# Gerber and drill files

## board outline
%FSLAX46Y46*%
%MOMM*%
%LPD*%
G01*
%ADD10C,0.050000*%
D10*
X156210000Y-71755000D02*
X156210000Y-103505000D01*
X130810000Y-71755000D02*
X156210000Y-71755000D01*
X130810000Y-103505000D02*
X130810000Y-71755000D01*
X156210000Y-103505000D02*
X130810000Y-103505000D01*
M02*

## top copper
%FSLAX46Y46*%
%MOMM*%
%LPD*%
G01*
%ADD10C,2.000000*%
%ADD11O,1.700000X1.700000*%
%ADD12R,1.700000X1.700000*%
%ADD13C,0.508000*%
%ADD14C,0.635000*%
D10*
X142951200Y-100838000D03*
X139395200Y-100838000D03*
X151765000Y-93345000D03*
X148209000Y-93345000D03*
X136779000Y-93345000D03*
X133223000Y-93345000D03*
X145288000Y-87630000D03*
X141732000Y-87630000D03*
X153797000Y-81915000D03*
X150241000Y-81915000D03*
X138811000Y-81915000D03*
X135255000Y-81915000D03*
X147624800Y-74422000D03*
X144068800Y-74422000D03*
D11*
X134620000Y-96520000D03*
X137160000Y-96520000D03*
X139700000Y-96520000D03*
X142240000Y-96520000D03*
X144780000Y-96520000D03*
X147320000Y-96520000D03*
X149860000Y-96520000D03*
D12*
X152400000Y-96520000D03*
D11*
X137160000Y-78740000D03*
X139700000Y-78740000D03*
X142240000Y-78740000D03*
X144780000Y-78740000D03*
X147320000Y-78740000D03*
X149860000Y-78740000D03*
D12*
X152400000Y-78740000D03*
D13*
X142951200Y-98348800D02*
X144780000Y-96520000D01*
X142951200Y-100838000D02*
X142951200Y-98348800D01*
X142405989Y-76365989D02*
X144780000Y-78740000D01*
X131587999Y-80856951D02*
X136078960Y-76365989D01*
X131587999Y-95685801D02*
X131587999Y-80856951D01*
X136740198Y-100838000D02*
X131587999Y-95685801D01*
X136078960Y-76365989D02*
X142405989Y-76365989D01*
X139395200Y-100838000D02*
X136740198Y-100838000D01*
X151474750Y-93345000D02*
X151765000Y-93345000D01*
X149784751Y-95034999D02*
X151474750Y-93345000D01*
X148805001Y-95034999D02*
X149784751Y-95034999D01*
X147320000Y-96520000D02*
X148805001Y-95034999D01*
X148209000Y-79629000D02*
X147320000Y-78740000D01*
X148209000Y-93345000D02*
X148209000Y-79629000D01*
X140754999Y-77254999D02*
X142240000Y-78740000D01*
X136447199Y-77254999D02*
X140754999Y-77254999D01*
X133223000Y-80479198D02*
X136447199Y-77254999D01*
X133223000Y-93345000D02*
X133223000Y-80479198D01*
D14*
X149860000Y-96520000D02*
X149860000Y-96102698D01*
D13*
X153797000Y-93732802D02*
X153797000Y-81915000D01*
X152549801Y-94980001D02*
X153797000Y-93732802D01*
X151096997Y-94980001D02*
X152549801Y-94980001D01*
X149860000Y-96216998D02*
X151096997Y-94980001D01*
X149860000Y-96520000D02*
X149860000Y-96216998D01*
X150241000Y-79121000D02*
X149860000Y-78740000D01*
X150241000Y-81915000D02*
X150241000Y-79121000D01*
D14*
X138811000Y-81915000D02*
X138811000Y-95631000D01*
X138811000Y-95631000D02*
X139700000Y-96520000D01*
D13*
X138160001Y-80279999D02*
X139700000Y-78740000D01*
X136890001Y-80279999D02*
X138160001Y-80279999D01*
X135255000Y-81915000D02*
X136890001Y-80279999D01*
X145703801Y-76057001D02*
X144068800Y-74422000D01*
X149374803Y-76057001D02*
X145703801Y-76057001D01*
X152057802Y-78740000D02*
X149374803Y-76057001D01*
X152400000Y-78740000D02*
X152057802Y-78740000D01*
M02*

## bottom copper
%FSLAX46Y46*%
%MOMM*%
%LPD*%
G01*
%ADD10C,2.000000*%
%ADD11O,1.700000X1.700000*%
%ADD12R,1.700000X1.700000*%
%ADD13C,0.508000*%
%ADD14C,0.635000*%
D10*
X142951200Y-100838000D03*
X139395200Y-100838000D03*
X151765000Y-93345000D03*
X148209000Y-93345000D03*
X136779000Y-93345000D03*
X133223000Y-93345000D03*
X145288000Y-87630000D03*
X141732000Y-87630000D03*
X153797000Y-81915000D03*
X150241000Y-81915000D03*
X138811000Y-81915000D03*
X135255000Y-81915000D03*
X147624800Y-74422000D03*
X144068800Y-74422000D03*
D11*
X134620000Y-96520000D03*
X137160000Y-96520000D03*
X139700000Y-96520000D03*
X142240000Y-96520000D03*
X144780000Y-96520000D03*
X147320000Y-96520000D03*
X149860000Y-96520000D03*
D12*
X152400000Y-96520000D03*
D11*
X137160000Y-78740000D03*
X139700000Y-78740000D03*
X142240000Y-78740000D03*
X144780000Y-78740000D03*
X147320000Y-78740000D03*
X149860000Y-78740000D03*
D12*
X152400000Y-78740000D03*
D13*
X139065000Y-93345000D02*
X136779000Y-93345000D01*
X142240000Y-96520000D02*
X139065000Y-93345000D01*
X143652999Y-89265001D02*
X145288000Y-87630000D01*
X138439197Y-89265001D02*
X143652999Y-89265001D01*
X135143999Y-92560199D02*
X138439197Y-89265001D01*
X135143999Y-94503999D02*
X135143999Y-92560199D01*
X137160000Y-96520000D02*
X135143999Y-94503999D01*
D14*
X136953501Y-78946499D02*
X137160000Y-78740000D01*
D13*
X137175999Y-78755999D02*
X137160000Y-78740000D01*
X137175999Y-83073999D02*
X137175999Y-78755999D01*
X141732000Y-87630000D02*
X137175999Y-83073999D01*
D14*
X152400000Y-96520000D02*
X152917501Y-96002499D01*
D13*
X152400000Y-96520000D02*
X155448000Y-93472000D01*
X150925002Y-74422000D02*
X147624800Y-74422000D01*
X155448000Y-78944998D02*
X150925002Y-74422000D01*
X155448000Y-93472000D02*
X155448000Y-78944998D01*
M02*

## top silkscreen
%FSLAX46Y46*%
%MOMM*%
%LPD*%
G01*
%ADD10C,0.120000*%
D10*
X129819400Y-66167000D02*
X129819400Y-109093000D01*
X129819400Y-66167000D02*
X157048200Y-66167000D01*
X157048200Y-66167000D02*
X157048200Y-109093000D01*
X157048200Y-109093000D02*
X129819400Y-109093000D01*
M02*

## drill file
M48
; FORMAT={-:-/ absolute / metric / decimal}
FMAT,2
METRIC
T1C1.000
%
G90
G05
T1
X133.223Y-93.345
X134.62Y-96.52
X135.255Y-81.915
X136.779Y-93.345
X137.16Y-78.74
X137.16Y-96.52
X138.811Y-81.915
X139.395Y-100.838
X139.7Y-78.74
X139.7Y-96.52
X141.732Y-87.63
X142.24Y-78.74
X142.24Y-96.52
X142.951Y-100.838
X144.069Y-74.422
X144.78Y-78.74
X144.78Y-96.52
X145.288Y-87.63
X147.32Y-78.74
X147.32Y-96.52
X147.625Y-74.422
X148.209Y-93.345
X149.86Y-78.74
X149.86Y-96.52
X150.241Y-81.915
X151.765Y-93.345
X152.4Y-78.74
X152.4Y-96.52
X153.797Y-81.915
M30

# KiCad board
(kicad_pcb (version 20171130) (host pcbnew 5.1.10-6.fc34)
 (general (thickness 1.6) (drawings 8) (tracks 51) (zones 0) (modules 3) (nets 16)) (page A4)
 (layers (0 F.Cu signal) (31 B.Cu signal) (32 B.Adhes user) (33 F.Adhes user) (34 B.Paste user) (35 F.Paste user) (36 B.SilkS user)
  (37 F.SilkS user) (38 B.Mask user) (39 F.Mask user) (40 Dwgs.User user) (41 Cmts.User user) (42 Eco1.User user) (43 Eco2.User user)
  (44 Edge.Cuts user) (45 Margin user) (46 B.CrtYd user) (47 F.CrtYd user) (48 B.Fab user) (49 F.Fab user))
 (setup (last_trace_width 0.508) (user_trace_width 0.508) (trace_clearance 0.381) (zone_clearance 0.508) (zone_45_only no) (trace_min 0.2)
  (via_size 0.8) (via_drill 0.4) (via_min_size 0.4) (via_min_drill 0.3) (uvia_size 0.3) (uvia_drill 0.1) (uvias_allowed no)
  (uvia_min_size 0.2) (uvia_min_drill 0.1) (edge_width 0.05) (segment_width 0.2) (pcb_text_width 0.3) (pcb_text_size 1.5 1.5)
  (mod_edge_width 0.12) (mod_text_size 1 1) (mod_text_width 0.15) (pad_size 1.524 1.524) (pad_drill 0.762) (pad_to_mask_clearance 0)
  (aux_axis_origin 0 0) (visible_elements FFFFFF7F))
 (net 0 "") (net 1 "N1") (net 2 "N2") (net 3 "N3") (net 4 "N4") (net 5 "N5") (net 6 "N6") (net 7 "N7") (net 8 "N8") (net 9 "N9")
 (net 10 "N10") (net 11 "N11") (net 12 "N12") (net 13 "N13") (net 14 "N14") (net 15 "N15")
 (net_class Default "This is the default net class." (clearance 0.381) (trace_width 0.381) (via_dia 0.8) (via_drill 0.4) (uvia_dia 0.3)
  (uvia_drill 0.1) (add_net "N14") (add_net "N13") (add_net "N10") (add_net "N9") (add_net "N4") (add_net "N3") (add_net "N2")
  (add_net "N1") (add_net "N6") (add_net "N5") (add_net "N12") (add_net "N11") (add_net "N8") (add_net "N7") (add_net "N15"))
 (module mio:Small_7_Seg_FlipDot (layer F.Cu) (at 143.51 87.63)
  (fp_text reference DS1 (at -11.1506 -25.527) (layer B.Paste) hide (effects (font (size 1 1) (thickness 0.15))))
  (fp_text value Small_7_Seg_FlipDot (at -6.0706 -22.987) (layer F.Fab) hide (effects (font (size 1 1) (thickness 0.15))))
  (fp_line (start -13.6906 -21.463) (end -13.6906 21.463) (layer F.SilkS) (width 0.12))
  (fp_line (start -13.6906 -21.463) (end 13.5382 -21.463) (layer F.SilkS) (width 0.12))
  (fp_line (start 13.5382 -21.463) (end 13.5382 21.463) (layer F.SilkS) (width 0.12))
  (fp_line (start 13.5382 21.463) (end -13.6906 21.463) (layer F.SilkS) (width 0.12))
  (pad D2 thru_hole circle (at -0.5588 13.208) (size 2 2) (drill 1) (layers *.Cu *.Mask) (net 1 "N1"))
  (pad D1 thru_hole circle (at -4.1148 13.208) (size 2 2) (drill 1) (layers *.Cu *.Mask) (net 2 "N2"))
  (pad C2 thru_hole circle (at 8.255 5.715) (size 2 2) (drill 1) (layers *.Cu *.Mask) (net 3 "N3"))
  (pad C1 thru_hole circle (at 4.699 5.715) (size 2 2) (drill 1) (layers *.Cu *.Mask) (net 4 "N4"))
  (pad E2 thru_hole circle (at -6.731 5.715) (size 2 2) (drill 1) (layers *.Cu *.Mask) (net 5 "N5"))
  (pad E1 thru_hole circle (at -10.287 5.715) (size 2 2) (drill 1) (layers *.Cu *.Mask) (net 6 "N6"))
  (pad G2 thru_hole circle (at 1.778 0) (size 2 2) (drill 1) (layers *.Cu *.Mask) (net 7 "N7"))
  (pad G1 thru_hole circle (at -1.778 0) (size 2 2) (drill 1) (layers *.Cu *.Mask) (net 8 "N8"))
  (pad B2 thru_hole circle (at 10.287 -5.715) (size 2 2) (drill 1) (layers *.Cu *.Mask) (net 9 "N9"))
  (pad B1 thru_hole circle (at 6.731 -5.715) (size 2 2) (drill 1) (layers *.Cu *.Mask) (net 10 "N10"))
  (pad F2 thru_hole circle (at -4.699 -5.715) (size 2 2) (drill 1) (layers *.Cu *.Mask) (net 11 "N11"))
  (pad F1 thru_hole circle (at -8.255 -5.715) (size 2 2) (drill 1) (layers *.Cu *.Mask) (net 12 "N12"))
  (pad A2 thru_hole circle (at 4.1148 -13.208) (size 2 2) (drill 1) (layers *.Cu *.Mask) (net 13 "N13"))
  (pad A1 thru_hole circle (at 0.5588 -13.208) (size 2 2) (drill 1) (layers *.Cu *.Mask) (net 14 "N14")))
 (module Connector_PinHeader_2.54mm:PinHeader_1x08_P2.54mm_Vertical (layer B.Cu) (at 152.4 96.52 90)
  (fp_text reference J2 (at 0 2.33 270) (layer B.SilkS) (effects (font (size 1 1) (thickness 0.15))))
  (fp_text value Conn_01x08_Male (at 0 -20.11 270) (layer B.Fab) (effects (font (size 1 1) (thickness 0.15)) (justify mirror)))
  (pad 8 thru_hole oval (at 0 -17.78 90) (size 1.7 1.7) (drill 1) (layers *.Cu *.Mask) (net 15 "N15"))
  (pad 7 thru_hole oval (at 0 -15.24 90) (size 1.7 1.7) (drill 1) (layers *.Cu *.Mask) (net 7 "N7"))
  (pad 6 thru_hole oval (at 0 -12.7 90) (size 1.7 1.7) (drill 1) (layers *.Cu *.Mask) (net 11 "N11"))
  (pad 5 thru_hole oval (at 0 -10.16 90) (size 1.7 1.7) (drill 1) (layers *.Cu *.Mask) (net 5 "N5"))
  (pad 4 thru_hole oval (at 0 -7.62 90) (size 1.7 1.7) (drill 1) (layers *.Cu *.Mask) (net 1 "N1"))
  (pad 3 thru_hole oval (at 0 -5.08 90) (size 1.7 1.7) (drill 1) (layers *.Cu *.Mask) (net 3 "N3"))
  (pad 2 thru_hole oval (at 0 -2.54 90) (size 1.7 1.7) (drill 1) (layers *.Cu *.Mask) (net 9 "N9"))
  (pad 1 thru_hole rect (at 0 0 90) (size 1.7 1.7) (drill 1) (layers *.Cu *.Mask) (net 13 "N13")))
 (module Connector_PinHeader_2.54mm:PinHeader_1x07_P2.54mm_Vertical (layer B.Cu) (at 152.4 78.74 90)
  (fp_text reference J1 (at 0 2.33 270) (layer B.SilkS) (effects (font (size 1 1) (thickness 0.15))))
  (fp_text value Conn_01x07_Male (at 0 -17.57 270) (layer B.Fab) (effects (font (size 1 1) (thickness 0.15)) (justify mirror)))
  (pad 7 thru_hole oval (at 0 -15.24 90) (size 1.7 1.7) (drill 1) (layers *.Cu *.Mask) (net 8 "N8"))
  (pad 6 thru_hole oval (at 0 -12.7 90) (size 1.7 1.7) (drill 1) (layers *.Cu *.Mask) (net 12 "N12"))
  (pad 5 thru_hole oval (at 0 -10.16 90) (size 1.7 1.7) (drill 1) (layers *.Cu *.Mask) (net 6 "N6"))
  (pad 4 thru_hole oval (at 0 -7.62 90) (size 1.7 1.7) (drill 1) (layers *.Cu *.Mask) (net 2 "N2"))
  (pad 3 thru_hole oval (at 0 -5.08 90) (size 1.7 1.7) (drill 1) (layers *.Cu *.Mask) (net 4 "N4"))
  (pad 2 thru_hole oval (at 0 -2.54 90) (size 1.7 1.7) (drill 1) (layers *.Cu *.Mask) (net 10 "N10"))
  (pad 1 thru_hole rect (at 0 0 90) (size 1.7 1.7) (drill 1) (layers *.Cu *.Mask) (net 14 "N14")))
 (gr_line (start 156.21 71.755) (end 156.21 103.505) (layer Edge.Cuts) (width 0.05))
 (gr_line (start 130.81 71.755) (end 156.21 71.755) (layer Edge.Cuts) (width 0.05))
 (gr_line (start 130.81 103.505) (end 130.81 71.755) (layer Edge.Cuts) (width 0.05))
 (gr_line (start 156.21 103.505) (end 130.81 103.505) (layer Edge.Cuts) (width 0.05))
 (segment (start 142.9512 98.3488) (end 144.78 96.52) (width 0.508) (layer F.Cu) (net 1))
 (segment (start 142.9512 100.838) (end 142.9512 98.3488) (width 0.508) (layer F.Cu) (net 1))
 (segment (start 142.405989 76.365989) (end 144.78 78.74) (width 0.508) (layer F.Cu) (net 2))
 (segment (start 131.587999 80.856951) (end 136.07896 76.365989) (width 0.508) (layer F.Cu) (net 2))
 (segment (start 131.587999 95.685801) (end 131.587999 80.856951) (width 0.508) (layer F.Cu) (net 2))
 (segment (start 136.740198 100.838) (end 131.587999 95.685801) (width 0.508) (layer F.Cu) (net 2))
 (segment (start 136.07896 76.365989) (end 142.405989 76.365989) (width 0.508) (layer F.Cu) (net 2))
 (segment (start 139.3952 100.838) (end 136.740198 100.838) (width 0.508) (layer F.Cu) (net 2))
 (segment (start 151.47475 93.345) (end 151.765 93.345) (width 0.508) (layer F.Cu) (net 3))
 (segment (start 149.784751 95.034999) (end 151.47475 93.345) (width 0.508) (layer F.Cu) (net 3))
 (segment (start 148.805001 95.034999) (end 149.784751 95.034999) (width 0.508) (layer F.Cu) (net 3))
 (segment (start 147.32 96.52) (end 148.805001 95.034999) (width 0.508) (layer F.Cu) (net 3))
 (segment (start 148.209 79.629) (end 147.32 78.74) (width 0.508) (layer F.Cu) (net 4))
 (segment (start 148.209 93.345) (end 148.209 79.629) (width 0.508) (layer F.Cu) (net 4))
 (segment (start 139.065 93.345) (end 136.779 93.345) (width 0.508) (layer B.Cu) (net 5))
 (segment (start 142.24 96.52) (end 139.065 93.345) (width 0.508) (layer B.Cu) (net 5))
 (segment (start 140.754999 77.254999) (end 142.24 78.74) (width 0.508) (layer F.Cu) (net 6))
 (segment (start 136.447199 77.254999) (end 140.754999 77.254999) (width 0.508) (layer F.Cu) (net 6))
 (segment (start 133.223 80.479198) (end 136.447199 77.254999) (width 0.508) (layer F.Cu) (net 6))
 (segment (start 133.223 93.345) (end 133.223 80.479198) (width 0.508) (layer F.Cu) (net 6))
 (segment (start 143.652999 89.265001) (end 145.288 87.63) (width 0.508) (layer B.Cu) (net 7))
 (segment (start 138.439197 89.265001) (end 143.652999 89.265001) (width 0.508) (layer B.Cu) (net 7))
 (segment (start 135.143999 92.560199) (end 138.439197 89.265001) (width 0.508) (layer B.Cu) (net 7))
 (segment (start 135.143999 94.503999) (end 135.143999 92.560199) (width 0.508) (layer B.Cu) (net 7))
 (segment (start 137.16 96.52) (end 135.143999 94.503999) (width 0.508) (layer B.Cu) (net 7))
 (segment (start 136.953501 78.946499) (end 137.16 78.74) (width 0.635) (layer B.Cu) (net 8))
 (segment (start 137.175999 78.755999) (end 137.16 78.74) (width 0.508) (layer B.Cu) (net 8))
 (segment (start 137.175999 83.073999) (end 137.175999 78.755999) (width 0.508) (layer B.Cu) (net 8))
 (segment (start 141.732 87.63) (end 137.175999 83.073999) (width 0.508) (layer B.Cu) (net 8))
 (segment (start 149.86 96.52) (end 149.86 96.102698) (width 0.635) (layer F.Cu) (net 9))
 (segment (start 153.797 93.732802) (end 153.797 81.915) (width 0.508) (layer F.Cu) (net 9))
 (segment (start 152.549801 94.980001) (end 153.797 93.732802) (width 0.508) (layer F.Cu) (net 9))
 (segment (start 151.096997 94.980001) (end 152.549801 94.980001) (width 0.508) (layer F.Cu) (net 9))
 (segment (start 149.86 96.216998) (end 151.096997 94.980001) (width 0.508) (layer F.Cu) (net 9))
 (segment (start 149.86 96.52) (end 149.86 96.216998) (width 0.508) (layer F.Cu) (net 9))
 (segment (start 150.241 79.121) (end 149.86 78.74) (width 0.508) (layer F.Cu) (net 10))
 (segment (start 150.241 81.915) (end 150.241 79.121) (width 0.508) (layer F.Cu) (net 10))
 (segment (start 138.811 81.915) (end 138.811 95.631) (width 0.635) (layer F.Cu) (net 11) (status 10))
 (segment (start 138.811 95.631) (end 139.7 96.52) (width 0.635) (layer F.Cu) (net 11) (status 20))
 (segment (start 138.160001 80.279999) (end 139.7 78.74) (width 0.508) (layer F.Cu) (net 12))
 (segment (start 136.890001 80.279999) (end 138.160001 80.279999) (width 0.508) (layer F.Cu) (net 12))
 (segment (start 135.255 81.915) (end 136.890001 80.279999) (width 0.508) (layer F.Cu) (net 12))
 (segment (start 152.4 96.52) (end 152.917501 96.002499) (width 0.635) (layer B.Cu) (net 13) (status 30))
 (segment (start 152.4 96.52) (end 155.448 93.472) (width 0.508) (layer B.Cu) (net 13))
 (segment (start 150.925002 74.422) (end 147.6248 74.422) (width 0.508) (layer B.Cu) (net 13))
 (segment (start 155.448 78.944998) (end 150.925002 74.422) (width 0.508) (layer B.Cu) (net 13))
 (segment (start 155.448 93.472) (end 155.448 78.944998) (width 0.508) (layer B.Cu) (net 13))
 (segment (start 145.703801 76.057001) (end 144.0688 74.422) (width 0.508) (layer F.Cu) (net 14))
 (segment (start 149.374803 76.057001) (end 145.703801 76.057001) (width 0.508) (layer F.Cu) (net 14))
 (segment (start 152.057802 78.74) (end 149.374803 76.057001) (width 0.508) (layer F.Cu) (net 14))
 (segment (start 152.4 78.74) (end 152.057802 78.74) (width 0.508) (layer F.Cu) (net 14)))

